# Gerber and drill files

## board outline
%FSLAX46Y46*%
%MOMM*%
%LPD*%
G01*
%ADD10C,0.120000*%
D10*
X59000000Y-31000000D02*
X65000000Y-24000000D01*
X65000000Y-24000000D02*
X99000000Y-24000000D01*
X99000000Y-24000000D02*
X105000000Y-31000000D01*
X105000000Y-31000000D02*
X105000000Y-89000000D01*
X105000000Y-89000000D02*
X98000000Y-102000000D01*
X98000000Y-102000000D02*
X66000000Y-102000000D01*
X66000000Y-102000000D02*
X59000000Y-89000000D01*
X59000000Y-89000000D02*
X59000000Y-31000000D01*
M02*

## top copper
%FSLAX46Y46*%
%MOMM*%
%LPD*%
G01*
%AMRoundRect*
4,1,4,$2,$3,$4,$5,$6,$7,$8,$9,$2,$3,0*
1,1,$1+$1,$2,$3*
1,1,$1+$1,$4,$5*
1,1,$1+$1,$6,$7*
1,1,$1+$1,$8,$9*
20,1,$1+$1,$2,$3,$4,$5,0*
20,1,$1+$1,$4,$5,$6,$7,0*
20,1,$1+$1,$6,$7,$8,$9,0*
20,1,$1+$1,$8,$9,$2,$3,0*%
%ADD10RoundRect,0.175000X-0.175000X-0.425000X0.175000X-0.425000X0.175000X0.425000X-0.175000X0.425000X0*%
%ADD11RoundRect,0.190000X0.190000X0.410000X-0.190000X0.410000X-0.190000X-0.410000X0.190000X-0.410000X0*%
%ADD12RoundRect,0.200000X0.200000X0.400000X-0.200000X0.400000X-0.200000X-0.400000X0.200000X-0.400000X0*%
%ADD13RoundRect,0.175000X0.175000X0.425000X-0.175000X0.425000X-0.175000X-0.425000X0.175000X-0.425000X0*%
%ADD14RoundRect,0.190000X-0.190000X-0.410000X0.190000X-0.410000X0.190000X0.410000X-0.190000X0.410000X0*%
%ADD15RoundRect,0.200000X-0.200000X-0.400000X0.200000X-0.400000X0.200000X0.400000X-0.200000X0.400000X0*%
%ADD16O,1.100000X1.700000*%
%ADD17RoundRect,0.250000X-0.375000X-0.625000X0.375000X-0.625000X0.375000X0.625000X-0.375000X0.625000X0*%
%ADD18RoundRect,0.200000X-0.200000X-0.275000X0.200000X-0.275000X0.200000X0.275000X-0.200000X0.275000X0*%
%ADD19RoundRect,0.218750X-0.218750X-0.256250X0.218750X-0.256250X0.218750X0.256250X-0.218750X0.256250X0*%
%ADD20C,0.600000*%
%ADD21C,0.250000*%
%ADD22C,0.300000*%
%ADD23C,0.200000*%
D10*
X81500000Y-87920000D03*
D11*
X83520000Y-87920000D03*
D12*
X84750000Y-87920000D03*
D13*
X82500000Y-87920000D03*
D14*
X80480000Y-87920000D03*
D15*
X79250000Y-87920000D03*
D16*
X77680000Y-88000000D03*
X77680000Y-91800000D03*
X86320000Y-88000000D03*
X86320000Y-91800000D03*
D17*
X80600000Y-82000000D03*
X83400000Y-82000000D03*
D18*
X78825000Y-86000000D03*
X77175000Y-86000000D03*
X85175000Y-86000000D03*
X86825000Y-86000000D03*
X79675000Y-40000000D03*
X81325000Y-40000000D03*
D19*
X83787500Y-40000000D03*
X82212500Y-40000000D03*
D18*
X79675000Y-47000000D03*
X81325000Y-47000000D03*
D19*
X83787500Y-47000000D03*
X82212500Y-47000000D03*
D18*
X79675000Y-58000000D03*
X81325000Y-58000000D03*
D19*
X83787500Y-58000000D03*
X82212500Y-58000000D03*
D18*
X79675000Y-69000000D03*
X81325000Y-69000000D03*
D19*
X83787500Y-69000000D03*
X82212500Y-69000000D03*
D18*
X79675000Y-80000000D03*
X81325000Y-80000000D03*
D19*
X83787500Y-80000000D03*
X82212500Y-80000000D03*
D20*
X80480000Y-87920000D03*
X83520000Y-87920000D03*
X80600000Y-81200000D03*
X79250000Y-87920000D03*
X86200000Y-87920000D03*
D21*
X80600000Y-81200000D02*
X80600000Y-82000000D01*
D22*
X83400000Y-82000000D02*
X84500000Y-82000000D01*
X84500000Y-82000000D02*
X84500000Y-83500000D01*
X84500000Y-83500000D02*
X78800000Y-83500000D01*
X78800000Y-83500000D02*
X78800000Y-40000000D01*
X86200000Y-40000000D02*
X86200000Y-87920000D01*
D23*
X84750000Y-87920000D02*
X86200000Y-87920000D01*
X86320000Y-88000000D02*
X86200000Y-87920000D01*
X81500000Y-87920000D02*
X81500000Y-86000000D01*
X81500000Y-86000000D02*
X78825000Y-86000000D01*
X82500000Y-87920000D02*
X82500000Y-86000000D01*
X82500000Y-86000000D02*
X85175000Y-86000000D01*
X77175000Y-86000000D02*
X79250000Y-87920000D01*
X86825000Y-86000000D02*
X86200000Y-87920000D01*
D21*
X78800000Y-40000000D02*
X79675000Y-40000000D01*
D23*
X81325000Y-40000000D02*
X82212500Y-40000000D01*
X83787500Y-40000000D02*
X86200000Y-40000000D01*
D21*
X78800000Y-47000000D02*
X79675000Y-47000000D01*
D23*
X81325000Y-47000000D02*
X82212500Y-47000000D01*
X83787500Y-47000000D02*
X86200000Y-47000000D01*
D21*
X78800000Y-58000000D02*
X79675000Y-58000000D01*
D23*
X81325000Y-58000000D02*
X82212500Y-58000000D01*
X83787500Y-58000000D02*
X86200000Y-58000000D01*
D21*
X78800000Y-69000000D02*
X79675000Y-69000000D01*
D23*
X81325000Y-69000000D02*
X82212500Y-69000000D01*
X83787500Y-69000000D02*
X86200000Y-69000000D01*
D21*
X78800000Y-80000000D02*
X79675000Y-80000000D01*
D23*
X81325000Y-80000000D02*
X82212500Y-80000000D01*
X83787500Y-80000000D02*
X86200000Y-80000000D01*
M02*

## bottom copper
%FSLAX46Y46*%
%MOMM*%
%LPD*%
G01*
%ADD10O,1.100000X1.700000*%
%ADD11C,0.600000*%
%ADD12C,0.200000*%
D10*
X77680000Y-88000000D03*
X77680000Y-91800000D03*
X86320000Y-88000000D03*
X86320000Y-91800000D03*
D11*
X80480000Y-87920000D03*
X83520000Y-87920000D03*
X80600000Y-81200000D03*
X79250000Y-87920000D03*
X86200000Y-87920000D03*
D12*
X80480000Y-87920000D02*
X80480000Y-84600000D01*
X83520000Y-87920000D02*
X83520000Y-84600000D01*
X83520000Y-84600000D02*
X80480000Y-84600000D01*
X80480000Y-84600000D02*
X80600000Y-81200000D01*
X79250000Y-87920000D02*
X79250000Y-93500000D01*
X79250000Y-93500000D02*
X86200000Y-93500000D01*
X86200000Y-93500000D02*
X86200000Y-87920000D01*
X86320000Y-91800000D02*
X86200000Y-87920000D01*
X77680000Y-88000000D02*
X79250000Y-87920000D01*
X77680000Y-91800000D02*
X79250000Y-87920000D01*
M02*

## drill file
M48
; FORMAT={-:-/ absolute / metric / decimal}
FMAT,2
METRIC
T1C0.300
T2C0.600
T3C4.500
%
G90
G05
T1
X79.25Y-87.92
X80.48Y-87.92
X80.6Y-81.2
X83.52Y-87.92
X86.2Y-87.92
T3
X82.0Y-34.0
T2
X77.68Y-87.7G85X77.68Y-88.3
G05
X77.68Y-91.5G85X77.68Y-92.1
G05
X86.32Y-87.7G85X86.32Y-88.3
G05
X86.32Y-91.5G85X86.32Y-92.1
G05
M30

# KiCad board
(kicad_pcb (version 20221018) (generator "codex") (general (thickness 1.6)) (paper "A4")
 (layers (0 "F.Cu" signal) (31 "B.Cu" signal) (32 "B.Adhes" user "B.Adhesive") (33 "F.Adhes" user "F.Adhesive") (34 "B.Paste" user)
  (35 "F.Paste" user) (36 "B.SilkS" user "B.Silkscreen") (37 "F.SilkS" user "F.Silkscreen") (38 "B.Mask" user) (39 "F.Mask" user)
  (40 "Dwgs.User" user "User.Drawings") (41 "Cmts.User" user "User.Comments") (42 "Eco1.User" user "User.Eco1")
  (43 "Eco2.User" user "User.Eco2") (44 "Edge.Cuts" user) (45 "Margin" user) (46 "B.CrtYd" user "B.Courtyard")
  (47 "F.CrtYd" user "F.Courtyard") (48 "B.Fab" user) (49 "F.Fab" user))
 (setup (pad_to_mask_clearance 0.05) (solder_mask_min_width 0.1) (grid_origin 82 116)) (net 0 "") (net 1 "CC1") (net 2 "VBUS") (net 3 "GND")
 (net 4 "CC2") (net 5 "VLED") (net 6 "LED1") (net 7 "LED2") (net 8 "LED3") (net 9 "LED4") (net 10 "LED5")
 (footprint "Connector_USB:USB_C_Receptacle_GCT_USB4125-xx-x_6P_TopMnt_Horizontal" (layer "F.Cu") (at 82 91)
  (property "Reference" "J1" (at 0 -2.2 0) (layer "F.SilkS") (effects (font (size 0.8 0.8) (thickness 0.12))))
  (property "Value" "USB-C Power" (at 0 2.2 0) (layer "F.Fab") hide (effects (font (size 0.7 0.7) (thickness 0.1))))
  (pad "A5" smd roundrect (at -0.5 -3.08) (size 0.7 1.2) (layers "F.Cu" "F.Paste" "F.Mask") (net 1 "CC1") (roundrect_rratio 0.25))
  (pad "A9" smd roundrect (at 1.52 -3.08 180) (size 0.76 1.2) (layers "F.Cu" "F.Paste" "F.Mask") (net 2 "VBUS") (roundrect_rratio 0.25))
  (pad "A12" smd roundrect (at 2.75 -3.08 180) (size 0.8 1.2) (layers "F.Cu" "F.Paste" "F.Mask") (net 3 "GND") (roundrect_rratio 0.25))
  (pad "B5" smd roundrect (at 0.5 -3.08 180) (size 0.7 1.2) (layers "F.Cu" "F.Paste" "F.Mask") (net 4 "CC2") (roundrect_rratio 0.25))
  (pad "B9" smd roundrect (at -1.52 -3.08) (size 0.76 1.2) (layers "F.Cu" "F.Paste" "F.Mask") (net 2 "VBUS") (roundrect_rratio 0.25))
  (pad "B12" smd roundrect (at -2.75 -3.08) (size 0.8 1.2) (layers "F.Cu" "F.Paste" "F.Mask") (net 3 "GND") (roundrect_rratio 0.25))
  (pad "SH" thru_hole oval (at -4.32 -3) (size 1.1 1.7) (drill oval 0.6 1.2) (layers "*.Cu" "*.Mask") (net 3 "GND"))
  (pad "SH" thru_hole oval (at -4.32 0.8) (size 1.1 1.7) (drill oval 0.6 1.2) (layers "*.Cu" "*.Mask") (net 3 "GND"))
  (pad "SH" thru_hole oval (at 4.32 -3) (size 1.1 1.7) (drill oval 0.6 1.2) (layers "*.Cu" "*.Mask") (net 3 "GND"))
  (pad "SH" thru_hole oval (at 4.32 0.8) (size 1.1 1.7) (drill oval 0.6 1.2) (layers "*.Cu" "*.Mask") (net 3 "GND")))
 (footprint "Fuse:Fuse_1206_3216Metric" (layer "F.Cu") (at 82 82)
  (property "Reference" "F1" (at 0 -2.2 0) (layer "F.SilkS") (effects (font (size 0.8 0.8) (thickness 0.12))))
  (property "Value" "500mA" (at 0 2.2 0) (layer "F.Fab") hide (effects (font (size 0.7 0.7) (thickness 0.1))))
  (pad "1" smd roundrect (at -1.4 0) (size 1.25 1.75) (layers "F.Cu" "F.Paste" "F.Mask") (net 2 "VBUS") (roundrect_rratio 0.2))
  (pad "2" smd roundrect (at 1.4 0) (size 1.25 1.75) (layers "F.Cu" "F.Paste" "F.Mask") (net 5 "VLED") (roundrect_rratio 0.2)))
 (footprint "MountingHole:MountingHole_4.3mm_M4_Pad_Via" (layer "F.Cu") (at 82 34)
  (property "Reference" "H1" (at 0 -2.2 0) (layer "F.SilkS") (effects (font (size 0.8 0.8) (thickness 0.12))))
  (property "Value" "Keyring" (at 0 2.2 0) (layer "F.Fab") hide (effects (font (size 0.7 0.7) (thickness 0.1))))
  (pad "1" np_thru_hole circle (at 0 0) (size 4.5 4.5) (drill 4.5) (layers "*.Cu" "*.Mask")))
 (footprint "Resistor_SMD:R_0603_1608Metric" (layer "F.Cu") (at 78 86 180)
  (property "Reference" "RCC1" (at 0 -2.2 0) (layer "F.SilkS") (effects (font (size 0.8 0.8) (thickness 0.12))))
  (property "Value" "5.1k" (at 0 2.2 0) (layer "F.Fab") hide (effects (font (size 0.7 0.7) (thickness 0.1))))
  (pad "1" smd roundrect (at -0.825 0) (size 0.8 0.95) (layers "F.Cu" "F.Paste" "F.Mask") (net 1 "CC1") (roundrect_rratio 0.25))
  (pad "2" smd roundrect (at 0.825 0) (size 0.8 0.95) (layers "F.Cu" "F.Paste" "F.Mask") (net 3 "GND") (roundrect_rratio 0.25)))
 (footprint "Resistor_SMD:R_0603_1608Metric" (layer "F.Cu") (at 86 86)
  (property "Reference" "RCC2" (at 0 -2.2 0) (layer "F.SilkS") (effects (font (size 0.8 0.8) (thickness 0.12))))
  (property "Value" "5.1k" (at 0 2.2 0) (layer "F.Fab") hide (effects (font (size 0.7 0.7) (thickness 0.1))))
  (pad "1" smd roundrect (at -0.825 0) (size 0.8 0.95) (layers "F.Cu" "F.Paste" "F.Mask") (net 4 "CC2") (roundrect_rratio 0.25))
  (pad "2" smd roundrect (at 0.825 0) (size 0.8 0.95) (layers "F.Cu" "F.Paste" "F.Mask") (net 3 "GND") (roundrect_rratio 0.25)))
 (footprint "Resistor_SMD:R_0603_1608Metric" (layer "F.Cu") (at 80.5 40 0)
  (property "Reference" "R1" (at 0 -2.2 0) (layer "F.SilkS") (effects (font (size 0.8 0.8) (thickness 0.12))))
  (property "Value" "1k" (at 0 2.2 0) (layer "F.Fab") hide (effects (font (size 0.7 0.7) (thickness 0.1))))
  (pad "1" smd roundrect (at -0.825 0) (size 0.8 0.95) (layers "F.Cu" "F.Paste" "F.Mask") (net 5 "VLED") (roundrect_rratio 0.25))
  (pad "2" smd roundrect (at 0.825 0) (size 0.8 0.95) (layers "F.Cu" "F.Paste" "F.Mask") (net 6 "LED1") (roundrect_rratio 0.25)))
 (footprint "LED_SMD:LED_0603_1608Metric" (layer "F.Cu") (at 83 40 180)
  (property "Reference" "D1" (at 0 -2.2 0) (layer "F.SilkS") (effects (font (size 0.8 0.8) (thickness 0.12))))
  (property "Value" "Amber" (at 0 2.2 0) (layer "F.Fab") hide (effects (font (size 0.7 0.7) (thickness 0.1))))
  (pad "1" smd roundrect (at -0.7875 0) (size 0.875 0.95) (layers "F.Cu" "F.Paste" "F.Mask") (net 3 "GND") (roundrect_rratio 0.25))
  (pad "2" smd roundrect (at 0.7875 0) (size 0.875 0.95) (layers "F.Cu" "F.Paste" "F.Mask") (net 6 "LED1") (roundrect_rratio 0.25)))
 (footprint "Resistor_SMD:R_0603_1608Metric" (layer "F.Cu") (at 80.5 47 0)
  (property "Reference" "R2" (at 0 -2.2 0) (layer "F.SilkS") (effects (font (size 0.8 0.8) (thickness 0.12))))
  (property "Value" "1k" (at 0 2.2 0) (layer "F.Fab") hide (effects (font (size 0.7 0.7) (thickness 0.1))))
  (pad "1" smd roundrect (at -0.825 0) (size 0.8 0.95) (layers "F.Cu" "F.Paste" "F.Mask") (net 5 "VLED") (roundrect_rratio 0.25))
  (pad "2" smd roundrect (at 0.825 0) (size 0.8 0.95) (layers "F.Cu" "F.Paste" "F.Mask") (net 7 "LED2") (roundrect_rratio 0.25)))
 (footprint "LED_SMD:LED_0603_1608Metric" (layer "F.Cu") (at 83 47 180)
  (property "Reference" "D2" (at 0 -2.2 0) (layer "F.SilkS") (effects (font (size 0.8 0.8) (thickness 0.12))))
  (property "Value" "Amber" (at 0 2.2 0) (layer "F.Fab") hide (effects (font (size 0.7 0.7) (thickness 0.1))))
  (pad "1" smd roundrect (at -0.7875 0) (size 0.875 0.95) (layers "F.Cu" "F.Paste" "F.Mask") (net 3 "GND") (roundrect_rratio 0.25))
  (pad "2" smd roundrect (at 0.7875 0) (size 0.875 0.95) (layers "F.Cu" "F.Paste" "F.Mask") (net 7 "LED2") (roundrect_rratio 0.25)))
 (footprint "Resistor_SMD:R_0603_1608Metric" (layer "F.Cu") (at 80.5 58 0)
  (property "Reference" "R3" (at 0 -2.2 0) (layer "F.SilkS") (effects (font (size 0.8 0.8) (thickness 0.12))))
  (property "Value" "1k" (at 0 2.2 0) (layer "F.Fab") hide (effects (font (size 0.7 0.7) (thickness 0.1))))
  (pad "1" smd roundrect (at -0.825 0) (size 0.8 0.95) (layers "F.Cu" "F.Paste" "F.Mask") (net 5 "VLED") (roundrect_rratio 0.25))
  (pad "2" smd roundrect (at 0.825 0) (size 0.8 0.95) (layers "F.Cu" "F.Paste" "F.Mask") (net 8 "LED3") (roundrect_rratio 0.25)))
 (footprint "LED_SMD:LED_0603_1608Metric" (layer "F.Cu") (at 83 58 180)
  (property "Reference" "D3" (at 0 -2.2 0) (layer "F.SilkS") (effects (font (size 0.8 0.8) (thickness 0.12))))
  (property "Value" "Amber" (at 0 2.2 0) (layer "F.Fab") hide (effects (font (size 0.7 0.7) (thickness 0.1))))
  (pad "1" smd roundrect (at -0.7875 0) (size 0.875 0.95) (layers "F.Cu" "F.Paste" "F.Mask") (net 3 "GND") (roundrect_rratio 0.25))
  (pad "2" smd roundrect (at 0.7875 0) (size 0.875 0.95) (layers "F.Cu" "F.Paste" "F.Mask") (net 8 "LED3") (roundrect_rratio 0.25)))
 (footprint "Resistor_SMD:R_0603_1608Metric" (layer "F.Cu") (at 80.5 69 0)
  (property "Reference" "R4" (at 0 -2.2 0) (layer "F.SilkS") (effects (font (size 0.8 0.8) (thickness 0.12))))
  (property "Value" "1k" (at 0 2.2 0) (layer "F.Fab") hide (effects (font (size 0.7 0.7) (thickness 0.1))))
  (pad "1" smd roundrect (at -0.825 0) (size 0.8 0.95) (layers "F.Cu" "F.Paste" "F.Mask") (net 5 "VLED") (roundrect_rratio 0.25))
  (pad "2" smd roundrect (at 0.825 0) (size 0.8 0.95) (layers "F.Cu" "F.Paste" "F.Mask") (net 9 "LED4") (roundrect_rratio 0.25)))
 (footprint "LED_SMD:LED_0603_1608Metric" (layer "F.Cu") (at 83 69 180)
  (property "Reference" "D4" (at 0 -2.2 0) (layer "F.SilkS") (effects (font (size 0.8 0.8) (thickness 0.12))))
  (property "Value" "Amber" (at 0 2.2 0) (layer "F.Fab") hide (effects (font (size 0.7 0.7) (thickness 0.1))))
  (pad "1" smd roundrect (at -0.7875 0) (size 0.875 0.95) (layers "F.Cu" "F.Paste" "F.Mask") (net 3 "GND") (roundrect_rratio 0.25))
  (pad "2" smd roundrect (at 0.7875 0) (size 0.875 0.95) (layers "F.Cu" "F.Paste" "F.Mask") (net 9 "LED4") (roundrect_rratio 0.25)))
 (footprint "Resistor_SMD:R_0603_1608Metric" (layer "F.Cu") (at 80.5 80 0)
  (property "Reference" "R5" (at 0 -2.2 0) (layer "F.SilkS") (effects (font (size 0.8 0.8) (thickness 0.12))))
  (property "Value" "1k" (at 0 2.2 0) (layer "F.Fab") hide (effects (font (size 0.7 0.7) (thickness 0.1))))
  (pad "1" smd roundrect (at -0.825 0) (size 0.8 0.95) (layers "F.Cu" "F.Paste" "F.Mask") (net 5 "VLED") (roundrect_rratio 0.25))
  (pad "2" smd roundrect (at 0.825 0) (size 0.8 0.95) (layers "F.Cu" "F.Paste" "F.Mask") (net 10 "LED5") (roundrect_rratio 0.25)))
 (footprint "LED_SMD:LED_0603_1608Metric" (layer "F.Cu") (at 83 80 180)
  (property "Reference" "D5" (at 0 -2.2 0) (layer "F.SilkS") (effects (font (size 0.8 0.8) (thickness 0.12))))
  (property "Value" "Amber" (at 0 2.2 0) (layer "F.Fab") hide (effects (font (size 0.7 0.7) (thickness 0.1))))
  (pad "1" smd roundrect (at -0.7875 0) (size 0.875 0.95) (layers "F.Cu" "F.Paste" "F.Mask") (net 3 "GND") (roundrect_rratio 0.25))
  (pad "2" smd roundrect (at 0.7875 0) (size 0.875 0.95) (layers "F.Cu" "F.Paste" "F.Mask") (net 10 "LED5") (roundrect_rratio 0.25)))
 (gr_line (start 59 31) (end 65 24) (stroke (width 0.12) (type solid)) (layer "Edge.Cuts"))
 (gr_line (start 65 24) (end 99 24) (stroke (width 0.12) (type solid)) (layer "Edge.Cuts"))
 (gr_line (start 99 24) (end 105 31) (stroke (width 0.12) (type solid)) (layer "Edge.Cuts"))
 (gr_line (start 105 31) (end 105 89) (stroke (width 0.12) (type solid)) (layer "Edge.Cuts"))
 (gr_line (start 105 89) (end 98 102) (stroke (width 0.12) (type solid)) (layer "Edge.Cuts"))
 (gr_line (start 98 102) (end 66 102) (stroke (width 0.12) (type solid)) (layer "Edge.Cuts"))
 (gr_line (start 66 102) (end 59 89) (stroke (width 0.12) (type solid)) (layer "Edge.Cuts"))
 (gr_line (start 59 89) (end 59 31) (stroke (width 0.12) (type solid)) (layer "Edge.Cuts"))
 (via (at 80.48 87.92) (size 0.6) (drill 0.3) (layers "F.Cu" "B.Cu") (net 2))
 (via (at 83.52 87.92) (size 0.6) (drill 0.3) (layers "F.Cu" "B.Cu") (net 2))
 (via (at 80.6 81.2) (size 0.6) (drill 0.3) (layers "F.Cu" "B.Cu") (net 2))
 (via (at 79.25 87.92) (size 0.6) (drill 0.3) (layers "F.Cu" "B.Cu") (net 3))
 (via (at 86.2 87.92) (size 0.6) (drill 0.3) (layers "F.Cu" "B.Cu") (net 3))
 (segment (start 80.6 81.2) (end 80.6 82.0) (width 0.25) (layer "F.Cu") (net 2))
 (segment (start 80.48 87.92) (end 80.48 84.6) (width 0.20) (layer "B.Cu") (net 2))
 (segment (start 83.52 87.92) (end 83.52 84.6) (width 0.20) (layer "B.Cu") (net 2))
 (segment (start 83.52 84.6) (end 80.48 84.6) (width 0.20) (layer "B.Cu") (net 2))
 (segment (start 80.48 84.6) (end 80.6 81.2) (width 0.20) (layer "B.Cu") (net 2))
 (segment (start 83.4 82.0) (end 84.5 82.0) (width 0.30) (layer "F.Cu") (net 5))
 (segment (start 84.5 82.0) (end 84.5 83.5) (width 0.30) (layer "F.Cu") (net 5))
 (segment (start 84.5 83.5) (end 78.8 83.5) (width 0.30) (layer "F.Cu") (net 5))
 (segment (start 78.8 83.5) (end 78.8 40.0) (width 0.30) (layer "F.Cu") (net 5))
 (segment (start 86.2 40.0) (end 86.2 87.92) (width 0.30) (layer "F.Cu") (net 3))
 (segment (start 84.75 87.92) (end 86.2 87.92) (width 0.20) (layer "F.Cu") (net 3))
 (segment (start 79.25 87.92) (end 79.25 93.5) (width 0.20) (layer "B.Cu") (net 3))
 (segment (start 79.25 93.5) (end 86.2 93.5) (width 0.20) (layer "B.Cu") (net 3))
 (segment (start 86.2 93.5) (end 86.2 87.92) (width 0.20) (layer "B.Cu") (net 3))
 (segment (start 86.32 88.0) (end 86.2 87.92) (width 0.20) (layer "F.Cu") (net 3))
 (segment (start 86.32 91.8) (end 86.2 87.92) (width 0.20) (layer "B.Cu") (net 3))
 (segment (start 77.68 88.0) (end 79.25 87.92) (width 0.20) (layer "B.Cu") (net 3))
 (segment (start 77.68 91.8) (end 79.25 87.92) (width 0.20) (layer "B.Cu") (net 3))
 (segment (start 81.5 87.92) (end 81.5 86.0) (width 0.20) (layer "F.Cu") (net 1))
 (segment (start 81.5 86.0) (end 78.825 86.0) (width 0.20) (layer "F.Cu") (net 1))
 (segment (start 82.5 87.92) (end 82.5 86.0) (width 0.20) (layer "F.Cu") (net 4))
 (segment (start 82.5 86.0) (end 85.175 86.0) (width 0.20) (layer "F.Cu") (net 4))
 (segment (start 77.175 86.0) (end 79.25 87.92) (width 0.20) (layer "F.Cu") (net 3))
 (segment (start 86.825 86.0) (end 86.2 87.92) (width 0.20) (layer "F.Cu") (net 3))
 (segment (start 78.8 40.0) (end 79.675 40.0) (width 0.25) (layer "F.Cu") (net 5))
 (segment (start 81.325 40.0) (end 82.2125 40.0) (width 0.20) (layer "F.Cu") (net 6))
 (segment (start 83.7875 40.0) (end 86.2 40.0) (width 0.20) (layer "F.Cu") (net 3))
 (segment (start 78.8 47.0) (end 79.675 47.0) (width 0.25) (layer "F.Cu") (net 5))
 (segment (start 81.325 47.0) (end 82.2125 47.0) (width 0.20) (layer "F.Cu") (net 7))
 (segment (start 83.7875 47.0) (end 86.2 47.0) (width 0.20) (layer "F.Cu") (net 3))
 (segment (start 78.8 58.0) (end 79.675 58.0) (width 0.25) (layer "F.Cu") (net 5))
 (segment (start 81.325 58.0) (end 82.2125 58.0) (width 0.20) (layer "F.Cu") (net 8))
 (segment (start 83.7875 58.0) (end 86.2 58.0) (width 0.20) (layer "F.Cu") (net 3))
 (segment (start 78.8 69.0) (end 79.675 69.0) (width 0.25) (layer "F.Cu") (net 5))
 (segment (start 81.325 69.0) (end 82.2125 69.0) (width 0.20) (layer "F.Cu") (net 9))
 (segment (start 83.7875 69.0) (end 86.2 69.0) (width 0.20) (layer "F.Cu") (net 3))
 (segment (start 78.8 80.0) (end 79.675 80.0) (width 0.25) (layer "F.Cu") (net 5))
 (segment (start 81.325 80.0) (end 82.2125 80.0) (width 0.20) (layer "F.Cu") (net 10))
 (segment (start 83.7875 80.0) (end 86.2 80.0) (width 0.20) (layer "F.Cu") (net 3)))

